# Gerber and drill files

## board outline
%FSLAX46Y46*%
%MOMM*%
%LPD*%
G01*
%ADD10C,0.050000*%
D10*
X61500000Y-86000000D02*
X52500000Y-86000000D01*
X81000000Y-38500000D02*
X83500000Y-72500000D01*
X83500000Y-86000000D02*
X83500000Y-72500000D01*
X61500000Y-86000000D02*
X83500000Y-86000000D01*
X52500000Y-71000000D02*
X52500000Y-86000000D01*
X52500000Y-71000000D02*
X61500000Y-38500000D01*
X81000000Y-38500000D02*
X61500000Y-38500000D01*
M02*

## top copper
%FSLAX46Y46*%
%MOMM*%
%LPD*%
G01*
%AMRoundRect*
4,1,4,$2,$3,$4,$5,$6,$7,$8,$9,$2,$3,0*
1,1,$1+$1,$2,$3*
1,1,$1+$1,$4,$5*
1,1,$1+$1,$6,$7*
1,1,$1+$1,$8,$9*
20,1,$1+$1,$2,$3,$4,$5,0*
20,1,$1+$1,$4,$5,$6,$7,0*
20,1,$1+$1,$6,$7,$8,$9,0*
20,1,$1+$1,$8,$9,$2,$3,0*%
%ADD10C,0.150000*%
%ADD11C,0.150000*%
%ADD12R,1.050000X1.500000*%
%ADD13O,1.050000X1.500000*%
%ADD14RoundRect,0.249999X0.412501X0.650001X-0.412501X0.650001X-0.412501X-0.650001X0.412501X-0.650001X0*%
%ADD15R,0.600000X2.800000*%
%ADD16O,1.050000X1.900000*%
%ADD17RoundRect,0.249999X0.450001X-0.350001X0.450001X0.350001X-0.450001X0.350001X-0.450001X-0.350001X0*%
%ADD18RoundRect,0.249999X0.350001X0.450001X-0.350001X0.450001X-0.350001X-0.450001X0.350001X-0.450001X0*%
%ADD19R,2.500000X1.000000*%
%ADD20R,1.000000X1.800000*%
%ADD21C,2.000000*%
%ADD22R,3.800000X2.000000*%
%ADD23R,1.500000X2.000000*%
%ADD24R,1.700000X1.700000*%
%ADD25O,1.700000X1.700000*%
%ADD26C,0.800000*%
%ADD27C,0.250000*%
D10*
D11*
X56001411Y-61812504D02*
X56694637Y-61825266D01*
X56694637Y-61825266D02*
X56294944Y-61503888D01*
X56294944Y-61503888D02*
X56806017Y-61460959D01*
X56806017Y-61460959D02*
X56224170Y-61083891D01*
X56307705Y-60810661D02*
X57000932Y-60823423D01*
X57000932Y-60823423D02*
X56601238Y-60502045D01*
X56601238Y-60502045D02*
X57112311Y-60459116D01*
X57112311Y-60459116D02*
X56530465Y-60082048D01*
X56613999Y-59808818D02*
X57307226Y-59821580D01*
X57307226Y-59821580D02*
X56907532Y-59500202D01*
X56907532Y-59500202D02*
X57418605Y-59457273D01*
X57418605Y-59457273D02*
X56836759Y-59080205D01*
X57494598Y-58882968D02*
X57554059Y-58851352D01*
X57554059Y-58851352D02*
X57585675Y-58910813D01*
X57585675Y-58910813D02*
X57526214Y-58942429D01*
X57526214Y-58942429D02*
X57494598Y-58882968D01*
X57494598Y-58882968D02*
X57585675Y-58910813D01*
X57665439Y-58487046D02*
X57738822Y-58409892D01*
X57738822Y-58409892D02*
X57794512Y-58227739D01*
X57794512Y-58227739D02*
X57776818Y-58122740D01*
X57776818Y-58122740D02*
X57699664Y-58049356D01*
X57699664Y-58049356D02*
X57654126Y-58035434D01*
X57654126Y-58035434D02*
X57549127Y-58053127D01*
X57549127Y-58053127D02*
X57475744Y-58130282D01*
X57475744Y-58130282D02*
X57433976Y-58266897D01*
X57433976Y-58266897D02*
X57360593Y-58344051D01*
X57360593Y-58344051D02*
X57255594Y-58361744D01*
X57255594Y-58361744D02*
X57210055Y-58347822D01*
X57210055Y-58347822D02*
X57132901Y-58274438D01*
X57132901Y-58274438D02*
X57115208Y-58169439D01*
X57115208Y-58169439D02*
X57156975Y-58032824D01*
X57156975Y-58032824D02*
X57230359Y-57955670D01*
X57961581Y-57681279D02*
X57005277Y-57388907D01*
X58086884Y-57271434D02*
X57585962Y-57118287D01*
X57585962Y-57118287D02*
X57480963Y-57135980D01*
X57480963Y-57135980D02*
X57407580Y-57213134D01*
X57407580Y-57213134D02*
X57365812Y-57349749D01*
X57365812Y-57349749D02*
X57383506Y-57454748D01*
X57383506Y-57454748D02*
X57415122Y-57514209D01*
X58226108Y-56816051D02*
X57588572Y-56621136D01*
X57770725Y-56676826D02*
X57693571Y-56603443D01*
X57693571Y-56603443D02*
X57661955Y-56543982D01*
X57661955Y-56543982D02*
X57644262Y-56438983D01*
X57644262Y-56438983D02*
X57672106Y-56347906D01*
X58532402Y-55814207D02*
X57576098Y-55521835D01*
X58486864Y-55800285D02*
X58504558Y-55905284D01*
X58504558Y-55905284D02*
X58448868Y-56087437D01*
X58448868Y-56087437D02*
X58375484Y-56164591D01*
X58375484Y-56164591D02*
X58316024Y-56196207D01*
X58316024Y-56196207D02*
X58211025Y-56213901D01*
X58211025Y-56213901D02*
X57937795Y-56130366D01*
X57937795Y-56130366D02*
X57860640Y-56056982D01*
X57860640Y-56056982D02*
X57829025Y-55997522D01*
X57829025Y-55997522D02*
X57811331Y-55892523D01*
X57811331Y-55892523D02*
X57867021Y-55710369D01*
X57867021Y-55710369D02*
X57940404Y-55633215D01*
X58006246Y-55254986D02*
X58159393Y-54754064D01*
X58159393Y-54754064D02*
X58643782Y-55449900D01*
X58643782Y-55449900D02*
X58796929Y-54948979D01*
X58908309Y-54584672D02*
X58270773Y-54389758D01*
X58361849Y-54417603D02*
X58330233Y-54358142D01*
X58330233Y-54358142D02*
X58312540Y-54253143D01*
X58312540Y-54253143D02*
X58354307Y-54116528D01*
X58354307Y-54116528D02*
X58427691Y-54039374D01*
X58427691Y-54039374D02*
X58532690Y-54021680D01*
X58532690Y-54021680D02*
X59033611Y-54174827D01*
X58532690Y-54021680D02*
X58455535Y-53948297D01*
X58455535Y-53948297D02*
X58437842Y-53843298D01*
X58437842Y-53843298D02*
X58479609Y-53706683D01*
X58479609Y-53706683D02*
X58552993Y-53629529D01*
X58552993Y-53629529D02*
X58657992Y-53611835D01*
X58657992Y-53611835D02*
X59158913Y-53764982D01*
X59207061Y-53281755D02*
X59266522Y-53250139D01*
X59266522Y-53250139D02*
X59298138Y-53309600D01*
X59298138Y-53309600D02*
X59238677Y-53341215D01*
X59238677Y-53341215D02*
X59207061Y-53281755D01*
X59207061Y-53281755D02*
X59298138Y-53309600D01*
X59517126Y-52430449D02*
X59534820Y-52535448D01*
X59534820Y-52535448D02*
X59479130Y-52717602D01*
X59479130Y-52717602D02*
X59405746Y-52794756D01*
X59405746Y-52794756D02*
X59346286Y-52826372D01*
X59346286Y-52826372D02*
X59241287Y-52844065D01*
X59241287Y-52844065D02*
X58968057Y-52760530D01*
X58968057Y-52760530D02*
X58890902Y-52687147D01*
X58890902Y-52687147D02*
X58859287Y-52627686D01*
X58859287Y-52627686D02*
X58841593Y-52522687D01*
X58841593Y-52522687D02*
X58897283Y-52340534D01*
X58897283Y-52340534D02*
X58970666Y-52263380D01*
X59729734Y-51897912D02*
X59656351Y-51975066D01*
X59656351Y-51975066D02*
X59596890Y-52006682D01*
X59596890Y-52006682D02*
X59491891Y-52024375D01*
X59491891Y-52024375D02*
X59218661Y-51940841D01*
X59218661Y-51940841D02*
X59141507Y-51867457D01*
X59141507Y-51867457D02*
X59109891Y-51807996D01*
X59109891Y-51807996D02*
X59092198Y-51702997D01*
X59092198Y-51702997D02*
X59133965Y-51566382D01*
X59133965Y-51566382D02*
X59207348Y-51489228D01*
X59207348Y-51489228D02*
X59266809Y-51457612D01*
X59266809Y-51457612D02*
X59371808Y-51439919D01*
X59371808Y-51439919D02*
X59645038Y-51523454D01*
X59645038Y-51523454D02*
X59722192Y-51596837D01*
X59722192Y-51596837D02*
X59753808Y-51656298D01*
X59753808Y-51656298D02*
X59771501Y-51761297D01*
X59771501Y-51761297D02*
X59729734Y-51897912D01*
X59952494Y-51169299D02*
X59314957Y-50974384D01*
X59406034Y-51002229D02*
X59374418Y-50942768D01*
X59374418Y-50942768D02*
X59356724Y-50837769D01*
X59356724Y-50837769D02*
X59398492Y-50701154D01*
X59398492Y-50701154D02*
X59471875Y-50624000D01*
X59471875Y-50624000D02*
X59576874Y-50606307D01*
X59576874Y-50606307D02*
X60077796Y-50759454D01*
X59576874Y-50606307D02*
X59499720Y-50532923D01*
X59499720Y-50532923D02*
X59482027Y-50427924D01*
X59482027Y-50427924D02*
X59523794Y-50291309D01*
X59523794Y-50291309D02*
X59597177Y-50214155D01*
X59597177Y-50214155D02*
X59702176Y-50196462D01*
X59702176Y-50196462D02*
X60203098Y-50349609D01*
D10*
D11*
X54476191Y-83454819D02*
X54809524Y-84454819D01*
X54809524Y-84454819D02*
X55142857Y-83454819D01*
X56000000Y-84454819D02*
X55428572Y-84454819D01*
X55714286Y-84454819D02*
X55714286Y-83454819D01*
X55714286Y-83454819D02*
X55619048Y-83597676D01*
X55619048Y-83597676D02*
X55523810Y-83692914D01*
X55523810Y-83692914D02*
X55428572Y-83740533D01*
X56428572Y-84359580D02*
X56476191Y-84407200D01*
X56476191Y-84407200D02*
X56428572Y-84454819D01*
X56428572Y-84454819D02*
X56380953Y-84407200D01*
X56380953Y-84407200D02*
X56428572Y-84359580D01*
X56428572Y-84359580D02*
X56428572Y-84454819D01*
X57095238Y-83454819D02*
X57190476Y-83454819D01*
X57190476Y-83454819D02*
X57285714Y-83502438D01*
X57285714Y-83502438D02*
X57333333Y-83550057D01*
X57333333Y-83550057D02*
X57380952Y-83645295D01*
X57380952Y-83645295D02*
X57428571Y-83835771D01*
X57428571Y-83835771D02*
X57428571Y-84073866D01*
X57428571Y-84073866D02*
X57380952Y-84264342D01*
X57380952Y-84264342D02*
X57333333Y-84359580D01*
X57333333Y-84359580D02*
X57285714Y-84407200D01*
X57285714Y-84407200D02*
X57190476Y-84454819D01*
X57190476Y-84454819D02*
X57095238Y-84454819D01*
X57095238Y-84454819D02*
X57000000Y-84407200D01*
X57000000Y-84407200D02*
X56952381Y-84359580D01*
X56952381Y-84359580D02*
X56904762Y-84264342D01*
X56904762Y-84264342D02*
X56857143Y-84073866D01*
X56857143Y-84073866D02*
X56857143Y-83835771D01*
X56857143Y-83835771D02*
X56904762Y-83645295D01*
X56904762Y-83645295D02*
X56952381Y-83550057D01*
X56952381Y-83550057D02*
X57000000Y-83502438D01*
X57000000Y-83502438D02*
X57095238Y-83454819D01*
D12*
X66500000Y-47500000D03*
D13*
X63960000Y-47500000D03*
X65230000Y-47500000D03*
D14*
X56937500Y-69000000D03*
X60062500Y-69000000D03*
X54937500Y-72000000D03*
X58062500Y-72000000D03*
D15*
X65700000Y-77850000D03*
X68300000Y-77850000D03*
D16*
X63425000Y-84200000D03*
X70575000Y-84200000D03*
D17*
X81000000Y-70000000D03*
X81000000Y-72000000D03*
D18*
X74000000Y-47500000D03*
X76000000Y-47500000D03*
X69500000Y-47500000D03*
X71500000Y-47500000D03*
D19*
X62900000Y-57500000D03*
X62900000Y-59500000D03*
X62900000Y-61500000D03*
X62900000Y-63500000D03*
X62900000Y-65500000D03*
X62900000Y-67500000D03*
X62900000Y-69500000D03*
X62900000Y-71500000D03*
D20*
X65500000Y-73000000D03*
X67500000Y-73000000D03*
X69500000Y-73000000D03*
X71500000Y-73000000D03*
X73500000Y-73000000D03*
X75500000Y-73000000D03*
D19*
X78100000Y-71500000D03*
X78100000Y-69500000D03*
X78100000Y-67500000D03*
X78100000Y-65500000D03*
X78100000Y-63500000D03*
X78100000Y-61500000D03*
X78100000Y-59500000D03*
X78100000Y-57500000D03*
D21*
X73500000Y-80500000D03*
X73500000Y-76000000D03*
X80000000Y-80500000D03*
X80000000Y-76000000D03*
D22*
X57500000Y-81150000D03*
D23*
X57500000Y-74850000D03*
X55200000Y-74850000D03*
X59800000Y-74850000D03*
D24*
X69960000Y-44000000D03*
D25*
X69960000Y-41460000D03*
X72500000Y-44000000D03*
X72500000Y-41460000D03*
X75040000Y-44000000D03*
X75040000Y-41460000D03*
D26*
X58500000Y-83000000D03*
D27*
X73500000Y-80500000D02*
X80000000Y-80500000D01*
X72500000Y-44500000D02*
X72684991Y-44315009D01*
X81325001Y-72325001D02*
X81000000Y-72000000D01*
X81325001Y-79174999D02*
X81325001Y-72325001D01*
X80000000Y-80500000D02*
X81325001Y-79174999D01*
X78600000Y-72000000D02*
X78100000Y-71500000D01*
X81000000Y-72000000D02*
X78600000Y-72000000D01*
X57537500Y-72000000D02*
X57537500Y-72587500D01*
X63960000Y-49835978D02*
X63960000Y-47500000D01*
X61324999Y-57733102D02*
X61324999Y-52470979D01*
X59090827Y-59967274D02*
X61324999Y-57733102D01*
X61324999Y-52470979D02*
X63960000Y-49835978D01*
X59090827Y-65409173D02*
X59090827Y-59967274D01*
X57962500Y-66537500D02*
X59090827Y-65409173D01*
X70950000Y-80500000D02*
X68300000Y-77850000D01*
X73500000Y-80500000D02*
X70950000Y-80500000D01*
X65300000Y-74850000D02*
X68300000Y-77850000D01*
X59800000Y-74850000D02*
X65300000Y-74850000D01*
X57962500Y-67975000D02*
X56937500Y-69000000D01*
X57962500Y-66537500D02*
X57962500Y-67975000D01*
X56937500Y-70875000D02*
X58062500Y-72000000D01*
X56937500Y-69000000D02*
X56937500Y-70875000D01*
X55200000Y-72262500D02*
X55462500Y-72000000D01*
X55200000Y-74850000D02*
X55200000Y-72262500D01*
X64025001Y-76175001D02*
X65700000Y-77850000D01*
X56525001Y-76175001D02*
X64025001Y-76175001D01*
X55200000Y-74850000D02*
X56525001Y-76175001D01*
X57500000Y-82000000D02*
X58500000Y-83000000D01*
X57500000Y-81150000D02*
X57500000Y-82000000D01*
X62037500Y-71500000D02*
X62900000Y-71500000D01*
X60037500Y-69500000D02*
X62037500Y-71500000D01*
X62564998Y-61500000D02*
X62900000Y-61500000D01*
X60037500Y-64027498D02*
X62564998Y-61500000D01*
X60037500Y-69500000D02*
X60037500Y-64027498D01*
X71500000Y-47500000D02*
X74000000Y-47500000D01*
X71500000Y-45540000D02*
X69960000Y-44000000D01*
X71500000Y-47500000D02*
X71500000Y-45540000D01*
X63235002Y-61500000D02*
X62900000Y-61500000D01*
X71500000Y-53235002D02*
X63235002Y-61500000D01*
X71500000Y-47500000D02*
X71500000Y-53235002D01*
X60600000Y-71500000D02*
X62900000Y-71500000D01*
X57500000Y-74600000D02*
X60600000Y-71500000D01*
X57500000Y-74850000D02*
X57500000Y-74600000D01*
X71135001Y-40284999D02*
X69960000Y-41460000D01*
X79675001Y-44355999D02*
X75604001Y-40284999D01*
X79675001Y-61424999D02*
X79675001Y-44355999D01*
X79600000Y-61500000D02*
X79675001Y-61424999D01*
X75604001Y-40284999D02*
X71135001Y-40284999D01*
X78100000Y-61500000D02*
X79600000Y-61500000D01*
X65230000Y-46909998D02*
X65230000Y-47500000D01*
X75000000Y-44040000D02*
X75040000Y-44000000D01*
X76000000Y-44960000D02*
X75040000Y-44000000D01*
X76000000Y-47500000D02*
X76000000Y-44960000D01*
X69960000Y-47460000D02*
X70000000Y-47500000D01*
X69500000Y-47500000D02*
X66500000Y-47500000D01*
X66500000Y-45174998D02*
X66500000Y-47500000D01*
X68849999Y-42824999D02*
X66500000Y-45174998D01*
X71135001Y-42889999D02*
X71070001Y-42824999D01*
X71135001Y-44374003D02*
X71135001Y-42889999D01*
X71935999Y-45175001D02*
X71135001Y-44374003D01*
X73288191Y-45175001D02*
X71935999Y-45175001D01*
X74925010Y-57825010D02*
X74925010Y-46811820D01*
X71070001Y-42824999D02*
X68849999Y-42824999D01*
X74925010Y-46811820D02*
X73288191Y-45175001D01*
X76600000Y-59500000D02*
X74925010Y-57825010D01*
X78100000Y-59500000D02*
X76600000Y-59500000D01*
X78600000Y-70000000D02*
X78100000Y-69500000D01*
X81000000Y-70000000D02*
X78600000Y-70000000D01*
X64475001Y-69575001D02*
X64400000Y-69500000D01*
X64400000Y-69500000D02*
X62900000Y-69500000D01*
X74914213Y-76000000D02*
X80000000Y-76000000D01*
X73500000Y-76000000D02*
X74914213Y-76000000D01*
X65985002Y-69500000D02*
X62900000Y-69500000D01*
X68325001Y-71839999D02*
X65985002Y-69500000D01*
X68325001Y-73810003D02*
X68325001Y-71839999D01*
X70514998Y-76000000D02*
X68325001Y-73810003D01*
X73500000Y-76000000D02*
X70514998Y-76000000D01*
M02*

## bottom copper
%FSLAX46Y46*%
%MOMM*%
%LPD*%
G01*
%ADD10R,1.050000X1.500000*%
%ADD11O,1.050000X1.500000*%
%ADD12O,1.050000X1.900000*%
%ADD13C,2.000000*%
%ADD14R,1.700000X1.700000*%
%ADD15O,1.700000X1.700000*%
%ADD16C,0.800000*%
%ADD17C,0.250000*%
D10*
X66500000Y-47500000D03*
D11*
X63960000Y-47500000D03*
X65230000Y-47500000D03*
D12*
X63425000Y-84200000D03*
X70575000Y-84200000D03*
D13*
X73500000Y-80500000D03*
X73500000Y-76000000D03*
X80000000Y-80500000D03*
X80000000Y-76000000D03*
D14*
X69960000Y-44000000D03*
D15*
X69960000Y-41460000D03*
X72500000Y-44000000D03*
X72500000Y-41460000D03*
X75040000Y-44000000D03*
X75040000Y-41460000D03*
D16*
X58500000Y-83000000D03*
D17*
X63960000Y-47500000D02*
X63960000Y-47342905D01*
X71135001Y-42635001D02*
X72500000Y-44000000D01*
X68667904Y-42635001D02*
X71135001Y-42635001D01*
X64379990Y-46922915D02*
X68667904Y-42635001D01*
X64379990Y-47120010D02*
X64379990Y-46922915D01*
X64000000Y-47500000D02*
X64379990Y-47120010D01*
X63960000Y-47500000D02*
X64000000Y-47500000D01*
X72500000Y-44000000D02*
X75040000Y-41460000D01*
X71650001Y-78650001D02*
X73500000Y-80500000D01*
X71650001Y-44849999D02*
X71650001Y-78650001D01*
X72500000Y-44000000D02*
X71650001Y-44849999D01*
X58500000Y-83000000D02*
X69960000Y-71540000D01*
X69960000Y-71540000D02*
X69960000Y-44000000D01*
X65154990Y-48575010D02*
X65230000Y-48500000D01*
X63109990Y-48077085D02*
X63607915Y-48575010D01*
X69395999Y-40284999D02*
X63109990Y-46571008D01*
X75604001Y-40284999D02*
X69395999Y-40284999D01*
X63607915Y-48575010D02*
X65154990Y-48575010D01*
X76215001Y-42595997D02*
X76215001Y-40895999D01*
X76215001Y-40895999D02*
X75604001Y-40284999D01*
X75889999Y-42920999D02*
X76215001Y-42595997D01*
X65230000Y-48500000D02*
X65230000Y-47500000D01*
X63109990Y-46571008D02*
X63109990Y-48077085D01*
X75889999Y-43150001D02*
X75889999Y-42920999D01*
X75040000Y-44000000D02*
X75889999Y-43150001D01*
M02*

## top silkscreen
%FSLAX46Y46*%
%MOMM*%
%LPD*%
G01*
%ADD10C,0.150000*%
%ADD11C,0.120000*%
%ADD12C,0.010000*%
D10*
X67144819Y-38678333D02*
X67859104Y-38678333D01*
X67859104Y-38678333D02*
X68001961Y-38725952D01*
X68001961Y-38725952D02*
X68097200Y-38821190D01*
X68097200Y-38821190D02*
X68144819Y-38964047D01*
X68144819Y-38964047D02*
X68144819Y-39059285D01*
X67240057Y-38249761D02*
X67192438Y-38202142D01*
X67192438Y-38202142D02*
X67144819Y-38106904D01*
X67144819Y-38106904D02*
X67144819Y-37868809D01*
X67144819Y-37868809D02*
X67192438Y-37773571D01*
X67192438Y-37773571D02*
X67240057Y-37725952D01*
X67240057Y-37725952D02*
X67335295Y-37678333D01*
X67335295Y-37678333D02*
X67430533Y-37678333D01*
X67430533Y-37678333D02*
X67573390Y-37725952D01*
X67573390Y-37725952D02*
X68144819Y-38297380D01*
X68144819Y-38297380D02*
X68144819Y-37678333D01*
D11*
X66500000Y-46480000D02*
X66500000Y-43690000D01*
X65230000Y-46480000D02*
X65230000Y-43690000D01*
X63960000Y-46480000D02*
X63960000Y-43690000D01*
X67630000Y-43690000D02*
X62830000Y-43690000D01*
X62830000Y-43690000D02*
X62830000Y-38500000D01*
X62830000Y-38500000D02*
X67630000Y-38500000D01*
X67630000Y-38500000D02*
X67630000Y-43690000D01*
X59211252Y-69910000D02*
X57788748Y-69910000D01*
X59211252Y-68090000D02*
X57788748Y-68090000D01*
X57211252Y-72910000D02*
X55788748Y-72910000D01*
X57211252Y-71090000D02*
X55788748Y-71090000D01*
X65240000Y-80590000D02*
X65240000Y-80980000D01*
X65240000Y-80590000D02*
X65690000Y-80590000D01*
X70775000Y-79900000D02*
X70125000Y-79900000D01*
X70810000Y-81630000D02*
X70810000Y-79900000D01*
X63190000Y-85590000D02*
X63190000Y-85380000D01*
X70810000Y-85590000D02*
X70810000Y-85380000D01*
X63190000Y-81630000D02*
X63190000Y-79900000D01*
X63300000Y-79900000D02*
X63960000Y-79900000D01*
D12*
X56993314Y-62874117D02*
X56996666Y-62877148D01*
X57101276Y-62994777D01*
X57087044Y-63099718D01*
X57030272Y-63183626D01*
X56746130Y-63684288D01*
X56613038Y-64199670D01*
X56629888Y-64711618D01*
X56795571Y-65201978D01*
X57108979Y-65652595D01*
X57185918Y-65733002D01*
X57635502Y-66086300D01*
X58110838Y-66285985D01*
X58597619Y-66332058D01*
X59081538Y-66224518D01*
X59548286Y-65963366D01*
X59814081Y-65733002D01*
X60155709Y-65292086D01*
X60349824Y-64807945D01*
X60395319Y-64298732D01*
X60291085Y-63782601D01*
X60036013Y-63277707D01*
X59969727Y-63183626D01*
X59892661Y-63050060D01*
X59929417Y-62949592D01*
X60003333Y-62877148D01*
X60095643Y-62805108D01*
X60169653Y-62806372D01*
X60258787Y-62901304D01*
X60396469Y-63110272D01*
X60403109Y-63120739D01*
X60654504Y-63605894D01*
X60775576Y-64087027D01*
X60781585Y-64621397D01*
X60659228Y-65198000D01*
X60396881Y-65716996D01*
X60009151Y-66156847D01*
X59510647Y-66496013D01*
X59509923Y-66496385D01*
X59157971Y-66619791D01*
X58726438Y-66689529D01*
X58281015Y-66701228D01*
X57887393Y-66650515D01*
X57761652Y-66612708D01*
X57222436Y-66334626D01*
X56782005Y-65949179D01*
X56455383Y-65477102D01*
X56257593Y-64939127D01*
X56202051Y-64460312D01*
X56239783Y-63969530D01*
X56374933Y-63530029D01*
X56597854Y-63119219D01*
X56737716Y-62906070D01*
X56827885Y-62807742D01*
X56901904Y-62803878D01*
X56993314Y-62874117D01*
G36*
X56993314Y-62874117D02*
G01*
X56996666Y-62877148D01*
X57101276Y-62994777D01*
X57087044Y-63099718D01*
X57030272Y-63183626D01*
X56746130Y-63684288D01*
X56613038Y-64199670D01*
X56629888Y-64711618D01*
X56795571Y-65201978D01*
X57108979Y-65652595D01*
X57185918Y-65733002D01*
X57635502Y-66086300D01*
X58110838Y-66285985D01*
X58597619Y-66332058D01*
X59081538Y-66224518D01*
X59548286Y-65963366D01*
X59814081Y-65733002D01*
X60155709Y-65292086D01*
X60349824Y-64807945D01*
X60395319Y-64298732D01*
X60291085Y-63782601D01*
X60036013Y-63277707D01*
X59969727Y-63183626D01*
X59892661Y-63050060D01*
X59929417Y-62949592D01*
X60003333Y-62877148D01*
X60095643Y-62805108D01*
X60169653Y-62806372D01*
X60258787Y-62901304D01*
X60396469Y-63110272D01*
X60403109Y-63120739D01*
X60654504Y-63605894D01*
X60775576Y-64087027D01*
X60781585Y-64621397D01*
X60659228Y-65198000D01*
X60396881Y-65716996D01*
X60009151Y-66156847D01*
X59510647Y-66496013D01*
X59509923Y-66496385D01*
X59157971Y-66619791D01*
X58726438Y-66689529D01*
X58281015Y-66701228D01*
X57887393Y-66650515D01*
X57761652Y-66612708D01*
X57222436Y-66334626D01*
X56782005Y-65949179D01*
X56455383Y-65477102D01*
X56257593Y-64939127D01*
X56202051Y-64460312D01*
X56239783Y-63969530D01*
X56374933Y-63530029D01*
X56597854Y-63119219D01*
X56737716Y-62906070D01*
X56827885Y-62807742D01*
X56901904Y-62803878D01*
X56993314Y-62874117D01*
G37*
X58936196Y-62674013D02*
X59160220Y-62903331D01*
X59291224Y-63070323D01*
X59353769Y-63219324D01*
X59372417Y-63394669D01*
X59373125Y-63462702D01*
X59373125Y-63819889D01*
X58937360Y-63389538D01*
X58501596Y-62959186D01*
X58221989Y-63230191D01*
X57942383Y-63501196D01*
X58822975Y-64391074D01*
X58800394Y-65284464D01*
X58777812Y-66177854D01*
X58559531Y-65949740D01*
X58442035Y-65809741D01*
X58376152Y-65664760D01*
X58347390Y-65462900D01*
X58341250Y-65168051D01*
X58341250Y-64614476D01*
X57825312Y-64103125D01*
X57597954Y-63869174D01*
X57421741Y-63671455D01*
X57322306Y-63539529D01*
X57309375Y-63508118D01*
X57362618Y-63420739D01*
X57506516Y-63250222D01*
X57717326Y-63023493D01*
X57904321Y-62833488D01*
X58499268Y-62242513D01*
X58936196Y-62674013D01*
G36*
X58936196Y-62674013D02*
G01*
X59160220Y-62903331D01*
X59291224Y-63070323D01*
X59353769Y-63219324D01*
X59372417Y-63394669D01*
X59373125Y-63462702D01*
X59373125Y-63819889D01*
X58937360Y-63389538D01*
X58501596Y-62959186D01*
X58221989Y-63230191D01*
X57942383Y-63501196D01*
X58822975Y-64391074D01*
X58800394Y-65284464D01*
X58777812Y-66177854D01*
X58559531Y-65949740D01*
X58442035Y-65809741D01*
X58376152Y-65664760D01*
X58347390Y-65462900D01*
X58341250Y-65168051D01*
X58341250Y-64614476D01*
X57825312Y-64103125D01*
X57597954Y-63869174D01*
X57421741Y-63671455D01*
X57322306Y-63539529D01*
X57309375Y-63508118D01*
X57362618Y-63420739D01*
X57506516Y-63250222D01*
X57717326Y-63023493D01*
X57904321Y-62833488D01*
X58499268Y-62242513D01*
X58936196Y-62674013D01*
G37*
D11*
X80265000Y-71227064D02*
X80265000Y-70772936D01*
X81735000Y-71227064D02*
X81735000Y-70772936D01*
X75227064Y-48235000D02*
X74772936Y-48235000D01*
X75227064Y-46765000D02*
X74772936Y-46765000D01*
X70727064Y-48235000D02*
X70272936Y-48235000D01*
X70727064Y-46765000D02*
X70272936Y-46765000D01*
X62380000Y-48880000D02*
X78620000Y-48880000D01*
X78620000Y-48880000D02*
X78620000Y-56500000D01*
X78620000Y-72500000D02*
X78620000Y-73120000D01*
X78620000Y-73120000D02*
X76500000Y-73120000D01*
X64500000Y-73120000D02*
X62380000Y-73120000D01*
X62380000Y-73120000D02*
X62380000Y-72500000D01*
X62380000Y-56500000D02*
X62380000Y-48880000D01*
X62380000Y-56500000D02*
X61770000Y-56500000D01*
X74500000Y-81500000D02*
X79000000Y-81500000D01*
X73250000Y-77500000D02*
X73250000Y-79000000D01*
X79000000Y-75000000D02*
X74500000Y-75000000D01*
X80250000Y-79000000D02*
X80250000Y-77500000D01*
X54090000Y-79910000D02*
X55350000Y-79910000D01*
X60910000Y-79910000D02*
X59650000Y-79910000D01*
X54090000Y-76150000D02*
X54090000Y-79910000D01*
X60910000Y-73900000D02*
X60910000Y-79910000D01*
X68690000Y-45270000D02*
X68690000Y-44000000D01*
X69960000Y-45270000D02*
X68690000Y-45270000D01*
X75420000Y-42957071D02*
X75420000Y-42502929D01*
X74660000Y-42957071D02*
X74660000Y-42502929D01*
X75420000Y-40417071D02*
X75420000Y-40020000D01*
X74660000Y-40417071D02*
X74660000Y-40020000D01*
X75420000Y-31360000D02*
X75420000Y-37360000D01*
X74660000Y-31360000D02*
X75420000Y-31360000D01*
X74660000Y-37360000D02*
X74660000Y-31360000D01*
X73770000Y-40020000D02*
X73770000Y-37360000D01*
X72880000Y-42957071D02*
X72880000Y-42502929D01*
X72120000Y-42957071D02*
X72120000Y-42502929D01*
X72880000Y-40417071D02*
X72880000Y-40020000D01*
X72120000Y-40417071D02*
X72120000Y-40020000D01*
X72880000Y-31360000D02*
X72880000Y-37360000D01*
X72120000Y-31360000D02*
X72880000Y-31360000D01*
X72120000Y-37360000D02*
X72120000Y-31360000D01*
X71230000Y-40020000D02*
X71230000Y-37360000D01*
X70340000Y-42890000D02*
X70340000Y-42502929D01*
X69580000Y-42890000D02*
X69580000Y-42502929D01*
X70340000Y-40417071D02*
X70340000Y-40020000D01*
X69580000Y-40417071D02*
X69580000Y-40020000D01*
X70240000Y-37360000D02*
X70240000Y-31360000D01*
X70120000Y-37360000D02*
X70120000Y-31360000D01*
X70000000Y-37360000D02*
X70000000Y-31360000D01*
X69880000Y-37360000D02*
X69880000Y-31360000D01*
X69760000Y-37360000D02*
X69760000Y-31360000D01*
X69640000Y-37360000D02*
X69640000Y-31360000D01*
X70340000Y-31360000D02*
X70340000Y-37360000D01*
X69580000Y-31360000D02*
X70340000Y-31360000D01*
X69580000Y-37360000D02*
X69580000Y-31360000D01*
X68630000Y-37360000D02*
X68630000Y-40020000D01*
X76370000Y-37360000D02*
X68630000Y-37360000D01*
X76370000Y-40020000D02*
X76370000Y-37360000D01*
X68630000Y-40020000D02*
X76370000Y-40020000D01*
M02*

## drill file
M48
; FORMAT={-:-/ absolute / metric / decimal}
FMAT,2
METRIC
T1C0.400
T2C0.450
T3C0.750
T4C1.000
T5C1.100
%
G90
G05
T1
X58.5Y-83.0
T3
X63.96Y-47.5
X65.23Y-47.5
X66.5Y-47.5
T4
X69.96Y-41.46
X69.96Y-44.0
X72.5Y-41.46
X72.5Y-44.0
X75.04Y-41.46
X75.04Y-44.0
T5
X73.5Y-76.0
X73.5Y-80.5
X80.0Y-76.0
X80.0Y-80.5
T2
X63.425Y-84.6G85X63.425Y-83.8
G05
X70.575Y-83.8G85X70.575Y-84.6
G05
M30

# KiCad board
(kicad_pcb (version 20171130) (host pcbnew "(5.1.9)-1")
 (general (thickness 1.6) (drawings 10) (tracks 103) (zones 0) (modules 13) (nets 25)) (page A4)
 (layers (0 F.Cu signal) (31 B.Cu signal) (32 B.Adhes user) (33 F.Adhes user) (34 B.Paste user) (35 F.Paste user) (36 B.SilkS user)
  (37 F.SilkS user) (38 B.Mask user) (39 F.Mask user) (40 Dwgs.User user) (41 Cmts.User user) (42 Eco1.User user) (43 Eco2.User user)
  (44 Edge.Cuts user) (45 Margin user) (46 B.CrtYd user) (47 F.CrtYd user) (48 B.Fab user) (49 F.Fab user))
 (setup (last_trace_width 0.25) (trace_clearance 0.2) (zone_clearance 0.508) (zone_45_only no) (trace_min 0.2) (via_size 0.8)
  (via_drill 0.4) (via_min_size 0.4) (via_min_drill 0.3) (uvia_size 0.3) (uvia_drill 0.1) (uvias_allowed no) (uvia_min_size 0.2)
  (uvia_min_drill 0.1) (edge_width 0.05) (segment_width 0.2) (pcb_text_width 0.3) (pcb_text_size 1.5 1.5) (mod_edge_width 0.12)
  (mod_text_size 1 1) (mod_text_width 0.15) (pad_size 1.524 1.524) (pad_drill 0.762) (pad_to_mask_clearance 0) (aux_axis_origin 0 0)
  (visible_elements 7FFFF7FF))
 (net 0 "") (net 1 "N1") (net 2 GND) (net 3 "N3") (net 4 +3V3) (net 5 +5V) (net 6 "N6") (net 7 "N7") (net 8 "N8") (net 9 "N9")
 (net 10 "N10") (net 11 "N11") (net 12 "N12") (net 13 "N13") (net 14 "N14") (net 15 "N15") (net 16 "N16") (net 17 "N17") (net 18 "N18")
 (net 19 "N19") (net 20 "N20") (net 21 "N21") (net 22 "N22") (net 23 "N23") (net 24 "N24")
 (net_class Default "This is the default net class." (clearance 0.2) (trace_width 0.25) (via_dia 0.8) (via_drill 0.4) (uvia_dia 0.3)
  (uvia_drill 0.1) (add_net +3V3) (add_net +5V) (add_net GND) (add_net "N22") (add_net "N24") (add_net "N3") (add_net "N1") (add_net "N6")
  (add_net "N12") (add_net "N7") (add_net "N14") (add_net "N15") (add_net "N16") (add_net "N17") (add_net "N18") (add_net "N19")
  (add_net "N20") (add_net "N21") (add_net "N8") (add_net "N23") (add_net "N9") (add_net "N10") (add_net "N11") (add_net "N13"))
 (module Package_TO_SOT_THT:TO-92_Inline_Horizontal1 (layer F.Cu) (at 66.5 47.5 180)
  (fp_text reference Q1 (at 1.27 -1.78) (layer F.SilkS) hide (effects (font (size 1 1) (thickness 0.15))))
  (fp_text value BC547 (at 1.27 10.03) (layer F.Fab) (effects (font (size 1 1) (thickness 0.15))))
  (fp_line (start 0 1.02) (end 0 3.81) (layer F.SilkS) (width 0.12))
  (fp_line (start 1.27 1.02) (end 1.27 3.81) (layer F.SilkS) (width 0.12))
  (fp_line (start 2.54 1.02) (end 2.54 3.81) (layer F.SilkS) (width 0.12))
  (fp_line (start -1.13 3.81) (end 3.67 3.81) (layer F.SilkS) (width 0.12))
  (fp_line (start 3.67 3.81) (end 3.67 9) (layer F.SilkS) (width 0.12))
  (fp_line (start 3.67 9) (end -1.13 9) (layer F.SilkS) (width 0.12))
  (fp_line (start -1.13 9) (end -1.13 3.81) (layer F.SilkS) (width 0.12))
  (pad 1 thru_hole rect (at 0 0 180) (size 1.05 1.5) (drill 0.75) (layers *.Cu *.Mask) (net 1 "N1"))
  (pad 3 thru_hole oval (at 2.54 0 180) (size 1.05 1.5) (drill 0.75) (layers *.Cu *.Mask) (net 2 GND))
  (pad 2 thru_hole oval (at 1.27 0 180) (size 1.05 1.5) (drill 0.75) (layers *.Cu *.Mask) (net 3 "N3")))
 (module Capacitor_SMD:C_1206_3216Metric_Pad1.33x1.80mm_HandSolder (layer F.Cu) (at 58.5 69 180)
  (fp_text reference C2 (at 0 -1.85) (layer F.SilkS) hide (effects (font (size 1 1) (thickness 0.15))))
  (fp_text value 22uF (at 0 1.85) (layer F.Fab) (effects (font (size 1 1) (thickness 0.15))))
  (fp_line (start -0.711252 -0.91) (end 0.711252 -0.91) (layer F.SilkS) (width 0.12))
  (fp_line (start -0.711252 0.91) (end 0.711252 0.91) (layer F.SilkS) (width 0.12))
  (pad 2 smd roundrect (at 1.5625 0 180) (size 1.325 1.8) (layers F.Cu F.Paste F.Mask) (roundrect_rratio 0.1886784905660377) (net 2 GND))
  (pad 1 smd roundrect (at -1.5625 0 180) (size 1.325 1.8) (layers F.Cu F.Paste F.Mask) (roundrect_rratio 0.1886784905660377) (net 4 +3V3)))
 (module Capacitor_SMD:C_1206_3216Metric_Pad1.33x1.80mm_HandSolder (layer F.Cu) (at 56.5 72 180)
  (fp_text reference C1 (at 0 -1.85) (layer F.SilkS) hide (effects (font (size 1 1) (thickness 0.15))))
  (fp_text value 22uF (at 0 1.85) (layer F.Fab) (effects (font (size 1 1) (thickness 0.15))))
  (fp_line (start -0.711252 -0.91) (end 0.711252 -0.91) (layer F.SilkS) (width 0.12))
  (fp_line (start -0.711252 0.91) (end 0.711252 0.91) (layer F.SilkS) (width 0.12))
  (pad 2 smd roundrect (at 1.5625 0 180) (size 1.325 1.8) (layers F.Cu F.Paste F.Mask) (roundrect_rratio 0.1886784905660377) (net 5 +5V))
  (pad 1 smd roundrect (at -1.5625 0 180) (size 1.325 1.8) (layers F.Cu F.Paste F.Mask) (roundrect_rratio 0.1886784905660377) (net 2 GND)))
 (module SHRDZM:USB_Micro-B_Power (layer F.Cu) (at 67 83)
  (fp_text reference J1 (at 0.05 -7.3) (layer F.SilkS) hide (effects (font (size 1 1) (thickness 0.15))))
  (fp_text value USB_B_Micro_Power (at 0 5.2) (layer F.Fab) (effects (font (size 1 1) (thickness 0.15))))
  (fp_line (start -1.76 -2.41) (end -1.76 -2.02) (layer F.SilkS) (width 0.12))
  (fp_line (start -1.76 -2.41) (end -1.31 -2.41) (layer F.SilkS) (width 0.12))
  (fp_line (start 3.775 -3.1) (end 3.125 -3.1) (layer F.SilkS) (width 0.12))
  (fp_line (start 3.81 -1.37) (end 3.81 -3.1) (layer F.SilkS) (width 0.12))
  (fp_line (start -3.81 2.59) (end -3.81 2.38) (layer F.SilkS) (width 0.12))
  (fp_line (start 3.81 2.59) (end 3.81 2.38) (layer F.SilkS) (width 0.12))
  (fp_line (start -3.81 -1.37) (end -3.81 -3.1) (layer F.SilkS) (width 0.12))
  (fp_line (start -3.7 -3.1) (end -3.04 -3.1) (layer F.SilkS) (width 0.12))
  (pad 1 smd rect (at -1.3 -5.15) (size 0.6 2.8) (layers F.Cu F.Paste F.Mask) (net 5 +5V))
  (pad 5 smd rect (at 1.3 -5.15) (size 0.6 2.8) (layers F.Cu F.Paste F.Mask) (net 2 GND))
  (pad "" thru_hole oval (at -3.575 1.2 180) (size 1.05 1.9) (drill oval 0.45 1.25) (layers *.Cu *.Mask))
  (pad "" thru_hole oval (at 3.575 1.2) (size 1.05 1.9) (drill oval 0.45 1.25) (layers *.Cu *.Mask)))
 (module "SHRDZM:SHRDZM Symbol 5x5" (layer F.Cu) (at 58.5 64.5)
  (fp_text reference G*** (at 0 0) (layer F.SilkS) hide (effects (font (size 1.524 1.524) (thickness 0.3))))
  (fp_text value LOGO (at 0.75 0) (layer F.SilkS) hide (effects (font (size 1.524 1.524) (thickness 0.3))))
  (fp_poly
   (pts (xy -1.506686 -1.625883) (xy -1.503334 -1.622852) (xy -1.398724 -1.505223) (xy -1.412956 -1.400282) (xy -1.469728 -1.316374)
    (xy -1.75387 -0.815712) (xy -1.886962 -0.30033) (xy -1.870112 0.211618) (xy -1.704429 0.701978) (xy -1.391021 1.152595)
    (xy -1.314082 1.233002) (xy -0.864498 1.5863) (xy -0.389162 1.785985) (xy 0.097619 1.832058) (xy 0.581538 1.724518)
    (xy 1.048286 1.463366) (xy 1.314081 1.233002) (xy 1.655709 0.792086) (xy 1.849824 0.307945) (xy 1.895319 -0.201268)
    (xy 1.791085 -0.717399) (xy 1.536013 -1.222293) (xy 1.469727 -1.316374) (xy 1.392661 -1.44994) (xy 1.429417 -1.550408)
    (xy 1.503333 -1.622852) (xy 1.595643 -1.694892) (xy 1.669653 -1.693628) (xy 1.758787 -1.598696) (xy 1.896469 -1.389728)
    (xy 1.903109 -1.379261) (xy 2.154504 -0.894106) (xy 2.275576 -0.412973) (xy 2.281585 0.121397) (xy 2.159228 0.698)
    (xy 1.896881 1.216996) (xy 1.509151 1.656847) (xy 1.010647 1.996013) (xy 1.009923 1.996385) (xy 0.657971 2.119791)
    (xy 0.226438 2.189529) (xy -0.218985 2.201228) (xy -0.612607 2.150515) (xy -0.738348 2.112708) (xy -1.277564 1.834626)
    (xy -1.717995 1.449179) (xy -2.044617 0.977102) (xy -2.242407 0.439127) (xy -2.297949 -0.039688) (xy -2.260217 -0.53047)
    (xy -2.125067 -0.969971) (xy -1.902146 -1.380781) (xy -1.762284 -1.59393) (xy -1.672115 -1.692258) (xy -1.598096 -1.696122)
    (xy -1.506686 -1.625883))
   (layer F.SilkS) (width 0.01))
  (fp_poly
   (pts (xy 0.436196 -1.825987) (xy 0.66022 -1.596669) (xy 0.791224 -1.429677) (xy 0.853769 -1.280676) (xy 0.872417 -1.105331)
    (xy 0.873125 -1.037298) (xy 0.873125 -0.680111) (xy 0.43736 -1.110462) (xy 0.001596 -1.540814) (xy -0.278011 -1.269809)
    (xy -0.557617 -0.998804) (xy 0.322975 -0.108926) (xy 0.300394 0.784464) (xy 0.277812 1.677854) (xy 0.059531 1.44974)
    (xy -0.057965 1.309741) (xy -0.123848 1.16476) (xy -0.15261 0.9629) (xy -0.15875 0.668051) (xy -0.15875 0.114476)
    (xy -0.674688 -0.396875) (xy -0.902046 -0.630826) (xy -1.078259 -0.828545) (xy -1.177694 -0.960471) (xy -1.190625 -0.991882)
    (xy -1.137382 -1.079261) (xy -0.993484 -1.249778) (xy -0.782674 -1.476507) (xy -0.595679 -1.666512) (xy -0.000732 -2.257487)
    (xy 0.436196 -1.825987))
   (layer F.SilkS) (width 0.01)))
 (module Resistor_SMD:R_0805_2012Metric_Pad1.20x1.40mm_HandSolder (layer F.Cu) (at 81 71 90)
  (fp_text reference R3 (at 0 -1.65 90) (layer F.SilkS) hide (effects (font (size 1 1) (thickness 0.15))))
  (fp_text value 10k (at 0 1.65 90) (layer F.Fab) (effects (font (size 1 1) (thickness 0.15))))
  (fp_line (start -0.227064 -0.735) (end 0.227064 -0.735) (layer F.SilkS) (width 0.12))
  (fp_line (start -0.227064 0.735) (end 0.227064 0.735) (layer F.SilkS) (width 0.12))
  (pad 2 smd roundrect (at 1 0 90) (size 1.2 1.4) (layers F.Cu F.Paste F.Mask) (roundrect_rratio 0.2083325) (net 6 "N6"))
  (pad 1 smd roundrect (at -1 0 90) (size 1.2 1.4) (layers F.Cu F.Paste F.Mask) (roundrect_rratio 0.2083325) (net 2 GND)))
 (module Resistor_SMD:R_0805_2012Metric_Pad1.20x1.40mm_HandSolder (layer F.Cu) (at 75 47.5 180)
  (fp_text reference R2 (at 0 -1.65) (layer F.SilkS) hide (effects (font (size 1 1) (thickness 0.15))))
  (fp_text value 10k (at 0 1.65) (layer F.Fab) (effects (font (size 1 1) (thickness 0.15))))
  (fp_line (start -0.227064 -0.735) (end 0.227064 -0.735) (layer F.SilkS) (width 0.12))
  (fp_line (start -0.227064 0.735) (end 0.227064 0.735) (layer F.SilkS) (width 0.12))
  (pad 2 smd roundrect (at 1 0 180) (size 1.2 1.4) (layers F.Cu F.Paste F.Mask) (roundrect_rratio 0.2083325) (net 4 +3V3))
  (pad 1 smd roundrect (at -1 0 180) (size 1.2 1.4) (layers F.Cu F.Paste F.Mask) (roundrect_rratio 0.2083325) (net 3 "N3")))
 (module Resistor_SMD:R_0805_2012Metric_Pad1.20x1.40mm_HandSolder (layer F.Cu) (at 70.5 47.5 180)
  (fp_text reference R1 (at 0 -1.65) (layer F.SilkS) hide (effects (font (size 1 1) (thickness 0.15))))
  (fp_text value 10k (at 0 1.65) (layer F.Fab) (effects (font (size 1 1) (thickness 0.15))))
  (fp_line (start -0.227064 -0.735) (end 0.227064 -0.735) (layer F.SilkS) (width 0.12))
  (fp_line (start -0.227064 0.735) (end 0.227064 0.735) (layer F.SilkS) (width 0.12))
  (pad 2 smd roundrect (at 1 0 180) (size 1.2 1.4) (layers F.Cu F.Paste F.Mask) (roundrect_rratio 0.2083325) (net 1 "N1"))
  (pad 1 smd roundrect (at -1 0 180) (size 1.2 1.4) (layers F.Cu F.Paste F.Mask) (roundrect_rratio 0.2083325) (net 4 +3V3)))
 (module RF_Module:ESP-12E (layer F.Cu) (at 70.5 61)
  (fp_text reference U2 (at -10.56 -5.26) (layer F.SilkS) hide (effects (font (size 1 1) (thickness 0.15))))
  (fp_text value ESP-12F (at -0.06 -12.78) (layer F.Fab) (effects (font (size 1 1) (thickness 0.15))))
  (fp_line (start -8.12 -12.12) (end 8.12 -12.12) (layer F.SilkS) (width 0.12))
  (fp_line (start 8.12 -12.12) (end 8.12 -4.5) (layer F.SilkS) (width 0.12))
  (fp_line (start 8.12 11.5) (end 8.12 12.12) (layer F.SilkS) (width 0.12))
  (fp_line (start 8.12 12.12) (end 6 12.12) (layer F.SilkS) (width 0.12))
  (fp_line (start -6 12.12) (end -8.12 12.12) (layer F.SilkS) (width 0.12))
  (fp_line (start -8.12 12.12) (end -8.12 11.5) (layer F.SilkS) (width 0.12))
  (fp_line (start -8.12 -4.5) (end -8.12 -12.12) (layer F.SilkS) (width 0.12))
  (fp_line (start -8.12 -4.5) (end -8.73 -4.5) (layer F.SilkS) (width 0.12))
  (pad 1 smd rect (at -7.6 -3.5) (size 2.5 1) (layers F.Cu F.Paste F.Mask) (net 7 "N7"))
  (pad 2 smd rect (at -7.6 -1.5) (size 2.5 1) (layers F.Cu F.Paste F.Mask) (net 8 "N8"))
  (pad 3 smd rect (at -7.6 0.5) (size 2.5 1) (layers F.Cu F.Paste F.Mask) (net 4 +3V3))
  (pad 4 smd rect (at -7.6 2.5) (size 2.5 1) (layers F.Cu F.Paste F.Mask) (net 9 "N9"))
  (pad 5 smd rect (at -7.6 4.5) (size 2.5 1) (layers F.Cu F.Paste F.Mask) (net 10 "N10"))
  (pad 6 smd rect (at -7.6 6.5) (size 2.5 1) (layers F.Cu F.Paste F.Mask) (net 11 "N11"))
  (pad 7 smd rect (at -7.6 8.5) (size 2.5 1) (layers F.Cu F.Paste F.Mask) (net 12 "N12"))
  (pad 8 smd rect (at -7.6 10.5) (size 2.5 1) (layers F.Cu F.Paste F.Mask) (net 4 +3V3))
  (pad 9 smd rect (at -5 12) (size 1 1.8) (layers F.Cu F.Paste F.Mask) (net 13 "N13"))
  (pad 10 smd rect (at -3 12) (size 1 1.8) (layers F.Cu F.Paste F.Mask) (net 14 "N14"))
  (pad 11 smd rect (at -1 12) (size 1 1.8) (layers F.Cu F.Paste F.Mask) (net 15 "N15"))
  (pad 12 smd rect (at 1 12) (size 1 1.8) (layers F.Cu F.Paste F.Mask) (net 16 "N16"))
  (pad 13 smd rect (at 3 12) (size 1 1.8) (layers F.Cu F.Paste F.Mask) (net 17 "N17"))
  (pad 14 smd rect (at 5 12) (size 1 1.8) (layers F.Cu F.Paste F.Mask) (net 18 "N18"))
  (pad 15 smd rect (at 7.6 10.5) (size 2.5 1) (layers F.Cu F.Paste F.Mask) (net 2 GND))
  (pad 16 smd rect (at 7.6 8.5) (size 2.5 1) (layers F.Cu F.Paste F.Mask) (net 6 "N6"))
  (pad 17 smd rect (at 7.6 6.5) (size 2.5 1) (layers F.Cu F.Paste F.Mask) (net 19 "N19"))
  (pad 18 smd rect (at 7.6 4.5) (size 2.5 1) (layers F.Cu F.Paste F.Mask) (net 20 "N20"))
  (pad 19 smd rect (at 7.6 2.5) (size 2.5 1) (layers F.Cu F.Paste F.Mask) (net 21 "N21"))
  (pad 20 smd rect (at 7.6 0.5) (size 2.5 1) (layers F.Cu F.Paste F.Mask) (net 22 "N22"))
  (pad 21 smd rect (at 7.6 -1.5) (size 2.5 1) (layers F.Cu F.Paste F.Mask) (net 1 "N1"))
  (pad 22 smd rect (at 7.6 -3.5) (size 2.5 1) (layers F.Cu F.Paste F.Mask) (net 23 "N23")))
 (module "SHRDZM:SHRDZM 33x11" (layer B.Cu) (at 66 65 270)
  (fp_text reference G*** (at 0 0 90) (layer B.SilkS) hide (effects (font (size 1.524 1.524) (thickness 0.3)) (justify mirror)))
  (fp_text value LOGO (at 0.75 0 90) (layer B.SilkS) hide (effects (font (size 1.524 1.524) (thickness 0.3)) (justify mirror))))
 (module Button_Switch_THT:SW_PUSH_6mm (layer F.Cu) (at 73.5 76)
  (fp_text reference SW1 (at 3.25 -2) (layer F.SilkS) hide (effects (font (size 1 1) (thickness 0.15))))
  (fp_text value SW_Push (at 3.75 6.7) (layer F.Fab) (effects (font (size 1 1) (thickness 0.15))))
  (fp_line (start 1 5.5) (end 5.5 5.5) (layer F.SilkS) (width 0.12))
  (fp_line (start -0.25 1.5) (end -0.25 3) (layer F.SilkS) (width 0.12))
  (fp_line (start 5.5 -1) (end 1 -1) (layer F.SilkS) (width 0.12))
  (fp_line (start 6.75 3) (end 6.75 1.5) (layer F.SilkS) (width 0.12))
  (pad 2 thru_hole circle (at 0 4.5 90) (size 2 2) (drill 1.1) (layers *.Cu *.Mask) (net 2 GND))
  (pad 1 thru_hole circle (at 0 0 90) (size 2 2) (drill 1.1) (layers *.Cu *.Mask) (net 12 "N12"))
  (pad 2 thru_hole circle (at 6.5 4.5 90) (size 2 2) (drill 1.1) (layers *.Cu *.Mask) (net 2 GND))
  (pad 1 thru_hole circle (at 6.5 0 90) (size 2 2) (drill 1.1) (layers *.Cu *.Mask) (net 12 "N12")))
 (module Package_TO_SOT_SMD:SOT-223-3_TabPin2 (layer F.Cu) (at 57.5 78 270)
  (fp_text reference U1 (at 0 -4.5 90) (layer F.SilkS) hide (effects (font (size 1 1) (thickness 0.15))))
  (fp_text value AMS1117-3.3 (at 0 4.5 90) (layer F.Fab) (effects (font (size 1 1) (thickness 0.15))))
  (fp_line (start 1.91 3.41) (end 1.91 2.15) (layer F.SilkS) (width 0.12))
  (fp_line (start 1.91 -3.41) (end 1.91 -2.15) (layer F.SilkS) (width 0.12))
  (fp_line (start -1.85 3.41) (end 1.91 3.41) (layer F.SilkS) (width 0.12))
  (fp_line (start -4.1 -3.41) (end 1.91 -3.41) (layer F.SilkS) (width 0.12))
  (pad 2 smd rect (at 3.15 0 270) (size 2 3.8) (layers F.Cu F.Paste F.Mask) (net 4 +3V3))
  (pad 2 smd rect (at -3.15 0 270) (size 2 1.5) (layers F.Cu F.Paste F.Mask) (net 4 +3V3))
  (pad 3 smd rect (at -3.15 2.3 270) (size 2 1.5) (layers F.Cu F.Paste F.Mask) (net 5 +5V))
  (pad 1 smd rect (at -3.15 -2.3 270) (size 2 1.5) (layers F.Cu F.Paste F.Mask) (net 2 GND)))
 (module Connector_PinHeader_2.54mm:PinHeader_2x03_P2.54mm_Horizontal (layer F.Cu) (at 69.96 44 90)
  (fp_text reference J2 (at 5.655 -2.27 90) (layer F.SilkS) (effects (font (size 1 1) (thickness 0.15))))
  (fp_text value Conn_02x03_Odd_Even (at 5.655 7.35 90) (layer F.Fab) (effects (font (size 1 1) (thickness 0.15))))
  (fp_line (start -1.27 -1.27) (end 0 -1.27) (layer F.SilkS) (width 0.12))
  (fp_line (start -1.27 0) (end -1.27 -1.27) (layer F.SilkS) (width 0.12))
  (fp_line (start 1.042929 5.46) (end 1.497071 5.46) (layer F.SilkS) (width 0.12))
  (fp_line (start 1.042929 4.7) (end 1.497071 4.7) (layer F.SilkS) (width 0.12))
  (fp_line (start 3.582929 5.46) (end 3.98 5.46) (layer F.SilkS) (width 0.12))
  (fp_line (start 3.582929 4.7) (end 3.98 4.7) (layer F.SilkS) (width 0.12))
  (fp_line (start 12.64 5.46) (end 6.64 5.46) (layer F.SilkS) (width 0.12))
  (fp_line (start 12.64 4.7) (end 12.64 5.46) (layer F.SilkS) (width 0.12))
  (fp_line (start 6.64 4.7) (end 12.64 4.7) (layer F.SilkS) (width 0.12))
  (fp_line (start 3.98 3.81) (end 6.64 3.81) (layer F.SilkS) (width 0.12))
  (fp_line (start 1.042929 2.92) (end 1.497071 2.92) (layer F.SilkS) (width 0.12))
  (fp_line (start 1.042929 2.16) (end 1.497071 2.16) (layer F.SilkS) (width 0.12))
  (fp_line (start 3.582929 2.92) (end 3.98 2.92) (layer F.SilkS) (width 0.12))
  (fp_line (start 3.582929 2.16) (end 3.98 2.16) (layer F.SilkS) (width 0.12))
  (fp_line (start 12.64 2.92) (end 6.64 2.92) (layer F.SilkS) (width 0.12))
  (fp_line (start 12.64 2.16) (end 12.64 2.92) (layer F.SilkS) (width 0.12))
  (fp_line (start 6.64 2.16) (end 12.64 2.16) (layer F.SilkS) (width 0.12))
  (fp_line (start 3.98 1.27) (end 6.64 1.27) (layer F.SilkS) (width 0.12))
  (fp_line (start 1.11 0.38) (end 1.497071 0.38) (layer F.SilkS) (width 0.12))
  (fp_line (start 1.11 -0.38) (end 1.497071 -0.38) (layer F.SilkS) (width 0.12))
  (fp_line (start 3.582929 0.38) (end 3.98 0.38) (layer F.SilkS) (width 0.12))
  (fp_line (start 3.582929 -0.38) (end 3.98 -0.38) (layer F.SilkS) (width 0.12))
  (fp_line (start 6.64 0.28) (end 12.64 0.28) (layer F.SilkS) (width 0.12))
  (fp_line (start 6.64 0.16) (end 12.64 0.16) (layer F.SilkS) (width 0.12))
  (fp_line (start 6.64 0.04) (end 12.64 0.04) (layer F.SilkS) (width 0.12))
  (fp_line (start 6.64 -0.08) (end 12.64 -0.08) (layer F.SilkS) (width 0.12))
  (fp_line (start 6.64 -0.2) (end 12.64 -0.2) (layer F.SilkS) (width 0.12))
  (fp_line (start 6.64 -0.32) (end 12.64 -0.32) (layer F.SilkS) (width 0.12))
  (fp_line (start 12.64 0.38) (end 6.64 0.38) (layer F.SilkS) (width 0.12))
  (fp_line (start 12.64 -0.38) (end 12.64 0.38) (layer F.SilkS) (width 0.12))
  (fp_line (start 6.64 -0.38) (end 12.64 -0.38) (layer F.SilkS) (width 0.12))
  (fp_line (start 6.64 -1.33) (end 3.98 -1.33) (layer F.SilkS) (width 0.12))
  (fp_line (start 6.64 6.41) (end 6.64 -1.33) (layer F.SilkS) (width 0.12))
  (fp_line (start 3.98 6.41) (end 6.64 6.41) (layer F.SilkS) (width 0.12))
  (fp_line (start 3.98 -1.33) (end 3.98 6.41) (layer F.SilkS) (width 0.12))
  (pad 1 thru_hole rect (at 0 0 90) (size 1.7 1.7) (drill 1) (layers *.Cu *.Mask) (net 4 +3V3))
  (pad 2 thru_hole oval (at 2.54 0 90) (size 1.7 1.7) (drill 1) (layers *.Cu *.Mask) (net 22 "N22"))
  (pad 3 thru_hole oval (at 0 2.54 90) (size 1.7 1.7) (drill 1) (layers *.Cu *.Mask) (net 2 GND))
  (pad 4 thru_hole oval (at 2.54 2.54 90) (size 1.7 1.7) (drill 1) (layers *.Cu *.Mask) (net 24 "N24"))
  (pad 5 thru_hole oval (at 0 5.08 90) (size 1.7 1.7) (drill 1) (layers *.Cu *.Mask) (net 3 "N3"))
  (pad 6 thru_hole oval (at 2.54 5.08 90) (size 1.7 1.7) (drill 1) (layers *.Cu *.Mask) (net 2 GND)))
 (gr_line (start 61.5 86) (end 52.5 86) (layer Edge.Cuts) (width 0.05))
 (gr_line (start 81 38.5) (end 83.5 72.5) (layer Edge.Cuts) (width 0.05))
 (gr_line (start 83.5 86) (end 83.5 72.5) (layer Edge.Cuts) (width 0.05))
 (gr_line (start 61.5 86) (end 83.5 86) (layer Edge.Cuts) (width 0.05))
 (gr_line (start 52.5 71) (end 52.5 86) (layer Edge.Cuts) (width 0.05))
 (gr_line (start 52.5 71) (end 61.5 38.5) (layer Edge.Cuts) (width 0.05))
 (gr_line (start 81 38.5) (end 61.5 38.5) (layer Edge.Cuts) (width 0.05))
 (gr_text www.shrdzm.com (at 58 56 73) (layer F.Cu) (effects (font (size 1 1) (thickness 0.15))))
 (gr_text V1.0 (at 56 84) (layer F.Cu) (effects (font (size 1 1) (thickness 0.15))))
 (segment (start 73.5 80.5) (end 80 80.5) (width 0.25) (layer F.Cu) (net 2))
 (segment (start 72.5 44.5) (end 72.684991 44.315009) (width 0.25) (layer F.Cu) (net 2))
 (segment (start 63.96 47.5) (end 63.96 47.342905) (width 0.25) (layer B.Cu) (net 2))
 (segment (start 81.325001 72.325001) (end 81 72) (width 0.25) (layer F.Cu) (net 2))
 (segment (start 81.325001 79.174999) (end 81.325001 72.325001) (width 0.25) (layer F.Cu) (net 2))
 (segment (start 80 80.5) (end 81.325001 79.174999) (width 0.25) (layer F.Cu) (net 2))
 (segment (start 78.6 72) (end 78.1 71.5) (width 0.25) (layer F.Cu) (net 2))
 (segment (start 81 72) (end 78.6 72) (width 0.25) (layer F.Cu) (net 2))
 (segment (start 57.5375 72) (end 57.5375 72.5875) (width 0.25) (layer F.Cu) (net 2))
 (segment (start 63.96 49.835978) (end 63.96 47.5) (width 0.25) (layer F.Cu) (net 2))
 (segment (start 61.324999 57.733102) (end 61.324999 52.470979) (width 0.25) (layer F.Cu) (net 2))
 (segment (start 59.090827 59.967274) (end 61.324999 57.733102) (width 0.25) (layer F.Cu) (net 2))
 (segment (start 61.324999 52.470979) (end 63.96 49.835978) (width 0.25) (layer F.Cu) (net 2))
 (segment (start 59.090827 65.409173) (end 59.090827 59.967274) (width 0.25) (layer F.Cu) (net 2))
 (segment (start 57.9625 66.5375) (end 59.090827 65.409173) (width 0.25) (layer F.Cu) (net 2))
 (segment (start 71.135001 42.635001) (end 72.5 44) (width 0.25) (layer B.Cu) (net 2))
 (segment (start 68.667904 42.635001) (end 71.135001 42.635001) (width 0.25) (layer B.Cu) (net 2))
 (segment (start 64.37999 46.922915) (end 68.667904 42.635001) (width 0.25) (layer B.Cu) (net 2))
 (segment (start 64.37999 47.12001) (end 64.37999 46.922915) (width 0.25) (layer B.Cu) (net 2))
 (segment (start 64 47.5) (end 64.37999 47.12001) (width 0.25) (layer B.Cu) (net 2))
 (segment (start 63.96 47.5) (end 64 47.5) (width 0.25) (layer B.Cu) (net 2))
 (segment (start 72.5 44) (end 75.04 41.46) (width 0.25) (layer B.Cu) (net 2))
 (segment (start 71.650001 78.650001) (end 73.5 80.5) (width 0.25) (layer B.Cu) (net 2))
 (segment (start 71.650001 44.849999) (end 71.650001 78.650001) (width 0.25) (layer B.Cu) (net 2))
 (segment (start 72.5 44) (end 71.650001 44.849999) (width 0.25) (layer B.Cu) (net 2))
 (segment (start 70.95 80.5) (end 68.3 77.85) (width 0.25) (layer F.Cu) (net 2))
 (segment (start 73.5 80.5) (end 70.95 80.5) (width 0.25) (layer F.Cu) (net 2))
 (segment (start 65.3 74.85) (end 68.3 77.85) (width 0.25) (layer F.Cu) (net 2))
 (segment (start 59.8 74.85) (end 65.3 74.85) (width 0.25) (layer F.Cu) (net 2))
 (segment (start 57.9625 67.975) (end 56.9375 69) (width 0.25) (layer F.Cu) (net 2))
 (segment (start 57.9625 66.5375) (end 57.9625 67.975) (width 0.25) (layer F.Cu) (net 2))
 (segment (start 56.9375 70.875) (end 58.0625 72) (width 0.25) (layer F.Cu) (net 2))
 (segment (start 56.9375 69) (end 56.9375 70.875) (width 0.25) (layer F.Cu) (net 2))
 (segment (start 55.2 72.2625) (end 55.4625 72) (width 0.25) (layer F.Cu) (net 5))
 (segment (start 55.2 74.85) (end 55.2 72.2625) (width 0.25) (layer F.Cu) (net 5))
 (segment (start 64.025001 76.175001) (end 65.7 77.85) (width 0.25) (layer F.Cu) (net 5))
 (segment (start 56.525001 76.175001) (end 64.025001 76.175001) (width 0.25) (layer F.Cu) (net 5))
 (segment (start 55.2 74.85) (end 56.525001 76.175001) (width 0.25) (layer F.Cu) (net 5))
 (via (at 58.5 83) (size 0.8) (drill 0.4) (layers F.Cu B.Cu) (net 4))
 (segment (start 57.5 82) (end 58.5 83) (width 0.25) (layer F.Cu) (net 4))
 (segment (start 57.5 81.15) (end 57.5 82) (width 0.25) (layer F.Cu) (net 4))
 (segment (start 62.0375 71.5) (end 62.9 71.5) (width 0.25) (layer F.Cu) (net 4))
 (segment (start 60.0375 69.5) (end 62.0375 71.5) (width 0.25) (layer F.Cu) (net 4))
 (segment (start 62.564998 61.5) (end 62.9 61.5) (width 0.25) (layer F.Cu) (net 4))
 (segment (start 60.0375 64.027498) (end 62.564998 61.5) (width 0.25) (layer F.Cu) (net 4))
 (segment (start 60.0375 69.5) (end 60.0375 64.027498) (width 0.25) (layer F.Cu) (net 4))
 (segment (start 71.5 47.5) (end 74 47.5) (width 0.25) (layer F.Cu) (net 4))
 (segment (start 71.5 45.54) (end 69.96 44) (width 0.25) (layer F.Cu) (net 4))
 (segment (start 71.5 47.5) (end 71.5 45.54) (width 0.25) (layer F.Cu) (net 4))
 (segment (start 63.235002 61.5) (end 62.9 61.5) (width 0.25) (layer F.Cu) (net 4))
 (segment (start 71.5 53.235002) (end 63.235002 61.5) (width 0.25) (layer F.Cu) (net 4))
 (segment (start 71.5 47.5) (end 71.5 53.235002) (width 0.25) (layer F.Cu) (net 4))
 (segment (start 58.5 83) (end 69.96 71.54) (width 0.25) (layer B.Cu) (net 4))
 (segment (start 60.6 71.5) (end 62.9 71.5) (width 0.25) (layer F.Cu) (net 4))
 (segment (start 57.5 74.6) (end 60.6 71.5) (width 0.25) (layer F.Cu) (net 4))
 (segment (start 57.5 74.85) (end 57.5 74.6) (width 0.25) (layer F.Cu) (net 4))
 (segment (start 69.96 71.54) (end 69.96 44) (width 0.25) (layer B.Cu) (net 4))
 (segment (start 71.135001 40.284999) (end 69.96 41.46) (width 0.25) (layer F.Cu) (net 22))
 (segment (start 79.675001 44.355999) (end 75.604001 40.284999) (width 0.25) (layer F.Cu) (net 22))
 (segment (start 79.675001 61.424999) (end 79.675001 44.355999) (width 0.25) (layer F.Cu) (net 22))
 (segment (start 79.6 61.5) (end 79.675001 61.424999) (width 0.25) (layer F.Cu) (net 22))
 (segment (start 75.604001 40.284999) (end 71.135001 40.284999) (width 0.25) (layer F.Cu) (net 22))
 (segment (start 78.1 61.5) (end 79.6 61.5) (width 0.25) (layer F.Cu) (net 22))
 (segment (start 65.23 46.909998) (end 65.23 47.5) (width 0.25) (layer F.Cu) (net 3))
 (segment (start 75 44.04) (end 75.04 44) (width 0.25) (layer F.Cu) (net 3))
 (segment (start 65.15499 48.57501) (end 65.23 48.5) (width 0.25) (layer B.Cu) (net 3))
 (segment (start 63.10999 48.077085) (end 63.607915 48.57501) (width 0.25) (layer B.Cu) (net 3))
 (segment (start 69.395999 40.284999) (end 63.10999 46.571008) (width 0.25) (layer B.Cu) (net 3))
 (segment (start 75.604001 40.284999) (end 69.395999 40.284999) (width 0.25) (layer B.Cu) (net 3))
 (segment (start 63.607915 48.57501) (end 65.15499 48.57501) (width 0.25) (layer B.Cu) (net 3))
 (segment (start 76.215001 42.595997) (end 76.215001 40.895999) (width 0.25) (layer B.Cu) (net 3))
 (segment (start 76.215001 40.895999) (end 75.604001 40.284999) (width 0.25) (layer B.Cu) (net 3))
 (segment (start 75.889999 42.920999) (end 76.215001 42.595997) (width 0.25) (layer B.Cu) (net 3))
 (segment (start 65.23 48.5) (end 65.23 47.5) (width 0.25) (layer B.Cu) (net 3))
 (segment (start 63.10999 46.571008) (end 63.10999 48.077085) (width 0.25) (layer B.Cu) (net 3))
 (segment (start 75.889999 43.150001) (end 75.889999 42.920999) (width 0.25) (layer B.Cu) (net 3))
 (segment (start 75.04 44) (end 75.889999 43.150001) (width 0.25) (layer B.Cu) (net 3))
 (segment (start 76 44.96) (end 75.04 44) (width 0.25) (layer F.Cu) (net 3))
 (segment (start 76 47.5) (end 76 44.96) (width 0.25) (layer F.Cu) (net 3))
 (segment (start 69.96 47.46) (end 70 47.5) (width 0.25) (layer F.Cu) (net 1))
 (segment (start 69.5 47.5) (end 66.5 47.5) (width 0.25) (layer F.Cu) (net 1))
 (segment (start 66.5 45.174998) (end 66.5 47.5) (width 0.25) (layer F.Cu) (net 1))
 (segment (start 68.849999 42.824999) (end 66.5 45.174998) (width 0.25) (layer F.Cu) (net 1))
 (segment (start 71.135001 42.889999) (end 71.070001 42.824999) (width 0.25) (layer F.Cu) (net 1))
 (segment (start 71.135001 44.374003) (end 71.135001 42.889999) (width 0.25) (layer F.Cu) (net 1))
 (segment (start 71.935999 45.175001) (end 71.135001 44.374003) (width 0.25) (layer F.Cu) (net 1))
 (segment (start 73.288191 45.175001) (end 71.935999 45.175001) (width 0.25) (layer F.Cu) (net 1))
 (segment (start 74.92501 57.82501) (end 74.92501 46.81182) (width 0.25) (layer F.Cu) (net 1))
 (segment (start 71.070001 42.824999) (end 68.849999 42.824999) (width 0.25) (layer F.Cu) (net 1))
 (segment (start 74.92501 46.81182) (end 73.288191 45.175001) (width 0.25) (layer F.Cu) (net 1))
 (segment (start 76.6 59.5) (end 74.92501 57.82501) (width 0.25) (layer F.Cu) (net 1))
 (segment (start 78.1 59.5) (end 76.6 59.5) (width 0.25) (layer F.Cu) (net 1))
 (segment (start 78.6 70) (end 78.1 69.5) (width 0.25) (layer F.Cu) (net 6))
 (segment (start 81 70) (end 78.6 70) (width 0.25) (layer F.Cu) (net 6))
 (segment (start 64.475001 69.575001) (end 64.4 69.5) (width 0.25) (layer F.Cu) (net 12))
 (segment (start 64.4 69.5) (end 62.9 69.5) (width 0.25) (layer F.Cu) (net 12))
 (segment (start 74.914213 76) (end 80 76) (width 0.25) (layer F.Cu) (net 12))
 (segment (start 73.5 76) (end 74.914213 76) (width 0.25) (layer F.Cu) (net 12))
 (segment (start 65.985002 69.5) (end 62.9 69.5) (width 0.25) (layer F.Cu) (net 12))
 (segment (start 68.325001 71.839999) (end 65.985002 69.5) (width 0.25) (layer F.Cu) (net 12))
 (segment (start 68.325001 73.810003) (end 68.325001 71.839999) (width 0.25) (layer F.Cu) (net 12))
 (segment (start 70.514998 76) (end 68.325001 73.810003) (width 0.25) (layer F.Cu) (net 12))
 (segment (start 73.5 76) (end 70.514998 76) (width 0.25) (layer F.Cu) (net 12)))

